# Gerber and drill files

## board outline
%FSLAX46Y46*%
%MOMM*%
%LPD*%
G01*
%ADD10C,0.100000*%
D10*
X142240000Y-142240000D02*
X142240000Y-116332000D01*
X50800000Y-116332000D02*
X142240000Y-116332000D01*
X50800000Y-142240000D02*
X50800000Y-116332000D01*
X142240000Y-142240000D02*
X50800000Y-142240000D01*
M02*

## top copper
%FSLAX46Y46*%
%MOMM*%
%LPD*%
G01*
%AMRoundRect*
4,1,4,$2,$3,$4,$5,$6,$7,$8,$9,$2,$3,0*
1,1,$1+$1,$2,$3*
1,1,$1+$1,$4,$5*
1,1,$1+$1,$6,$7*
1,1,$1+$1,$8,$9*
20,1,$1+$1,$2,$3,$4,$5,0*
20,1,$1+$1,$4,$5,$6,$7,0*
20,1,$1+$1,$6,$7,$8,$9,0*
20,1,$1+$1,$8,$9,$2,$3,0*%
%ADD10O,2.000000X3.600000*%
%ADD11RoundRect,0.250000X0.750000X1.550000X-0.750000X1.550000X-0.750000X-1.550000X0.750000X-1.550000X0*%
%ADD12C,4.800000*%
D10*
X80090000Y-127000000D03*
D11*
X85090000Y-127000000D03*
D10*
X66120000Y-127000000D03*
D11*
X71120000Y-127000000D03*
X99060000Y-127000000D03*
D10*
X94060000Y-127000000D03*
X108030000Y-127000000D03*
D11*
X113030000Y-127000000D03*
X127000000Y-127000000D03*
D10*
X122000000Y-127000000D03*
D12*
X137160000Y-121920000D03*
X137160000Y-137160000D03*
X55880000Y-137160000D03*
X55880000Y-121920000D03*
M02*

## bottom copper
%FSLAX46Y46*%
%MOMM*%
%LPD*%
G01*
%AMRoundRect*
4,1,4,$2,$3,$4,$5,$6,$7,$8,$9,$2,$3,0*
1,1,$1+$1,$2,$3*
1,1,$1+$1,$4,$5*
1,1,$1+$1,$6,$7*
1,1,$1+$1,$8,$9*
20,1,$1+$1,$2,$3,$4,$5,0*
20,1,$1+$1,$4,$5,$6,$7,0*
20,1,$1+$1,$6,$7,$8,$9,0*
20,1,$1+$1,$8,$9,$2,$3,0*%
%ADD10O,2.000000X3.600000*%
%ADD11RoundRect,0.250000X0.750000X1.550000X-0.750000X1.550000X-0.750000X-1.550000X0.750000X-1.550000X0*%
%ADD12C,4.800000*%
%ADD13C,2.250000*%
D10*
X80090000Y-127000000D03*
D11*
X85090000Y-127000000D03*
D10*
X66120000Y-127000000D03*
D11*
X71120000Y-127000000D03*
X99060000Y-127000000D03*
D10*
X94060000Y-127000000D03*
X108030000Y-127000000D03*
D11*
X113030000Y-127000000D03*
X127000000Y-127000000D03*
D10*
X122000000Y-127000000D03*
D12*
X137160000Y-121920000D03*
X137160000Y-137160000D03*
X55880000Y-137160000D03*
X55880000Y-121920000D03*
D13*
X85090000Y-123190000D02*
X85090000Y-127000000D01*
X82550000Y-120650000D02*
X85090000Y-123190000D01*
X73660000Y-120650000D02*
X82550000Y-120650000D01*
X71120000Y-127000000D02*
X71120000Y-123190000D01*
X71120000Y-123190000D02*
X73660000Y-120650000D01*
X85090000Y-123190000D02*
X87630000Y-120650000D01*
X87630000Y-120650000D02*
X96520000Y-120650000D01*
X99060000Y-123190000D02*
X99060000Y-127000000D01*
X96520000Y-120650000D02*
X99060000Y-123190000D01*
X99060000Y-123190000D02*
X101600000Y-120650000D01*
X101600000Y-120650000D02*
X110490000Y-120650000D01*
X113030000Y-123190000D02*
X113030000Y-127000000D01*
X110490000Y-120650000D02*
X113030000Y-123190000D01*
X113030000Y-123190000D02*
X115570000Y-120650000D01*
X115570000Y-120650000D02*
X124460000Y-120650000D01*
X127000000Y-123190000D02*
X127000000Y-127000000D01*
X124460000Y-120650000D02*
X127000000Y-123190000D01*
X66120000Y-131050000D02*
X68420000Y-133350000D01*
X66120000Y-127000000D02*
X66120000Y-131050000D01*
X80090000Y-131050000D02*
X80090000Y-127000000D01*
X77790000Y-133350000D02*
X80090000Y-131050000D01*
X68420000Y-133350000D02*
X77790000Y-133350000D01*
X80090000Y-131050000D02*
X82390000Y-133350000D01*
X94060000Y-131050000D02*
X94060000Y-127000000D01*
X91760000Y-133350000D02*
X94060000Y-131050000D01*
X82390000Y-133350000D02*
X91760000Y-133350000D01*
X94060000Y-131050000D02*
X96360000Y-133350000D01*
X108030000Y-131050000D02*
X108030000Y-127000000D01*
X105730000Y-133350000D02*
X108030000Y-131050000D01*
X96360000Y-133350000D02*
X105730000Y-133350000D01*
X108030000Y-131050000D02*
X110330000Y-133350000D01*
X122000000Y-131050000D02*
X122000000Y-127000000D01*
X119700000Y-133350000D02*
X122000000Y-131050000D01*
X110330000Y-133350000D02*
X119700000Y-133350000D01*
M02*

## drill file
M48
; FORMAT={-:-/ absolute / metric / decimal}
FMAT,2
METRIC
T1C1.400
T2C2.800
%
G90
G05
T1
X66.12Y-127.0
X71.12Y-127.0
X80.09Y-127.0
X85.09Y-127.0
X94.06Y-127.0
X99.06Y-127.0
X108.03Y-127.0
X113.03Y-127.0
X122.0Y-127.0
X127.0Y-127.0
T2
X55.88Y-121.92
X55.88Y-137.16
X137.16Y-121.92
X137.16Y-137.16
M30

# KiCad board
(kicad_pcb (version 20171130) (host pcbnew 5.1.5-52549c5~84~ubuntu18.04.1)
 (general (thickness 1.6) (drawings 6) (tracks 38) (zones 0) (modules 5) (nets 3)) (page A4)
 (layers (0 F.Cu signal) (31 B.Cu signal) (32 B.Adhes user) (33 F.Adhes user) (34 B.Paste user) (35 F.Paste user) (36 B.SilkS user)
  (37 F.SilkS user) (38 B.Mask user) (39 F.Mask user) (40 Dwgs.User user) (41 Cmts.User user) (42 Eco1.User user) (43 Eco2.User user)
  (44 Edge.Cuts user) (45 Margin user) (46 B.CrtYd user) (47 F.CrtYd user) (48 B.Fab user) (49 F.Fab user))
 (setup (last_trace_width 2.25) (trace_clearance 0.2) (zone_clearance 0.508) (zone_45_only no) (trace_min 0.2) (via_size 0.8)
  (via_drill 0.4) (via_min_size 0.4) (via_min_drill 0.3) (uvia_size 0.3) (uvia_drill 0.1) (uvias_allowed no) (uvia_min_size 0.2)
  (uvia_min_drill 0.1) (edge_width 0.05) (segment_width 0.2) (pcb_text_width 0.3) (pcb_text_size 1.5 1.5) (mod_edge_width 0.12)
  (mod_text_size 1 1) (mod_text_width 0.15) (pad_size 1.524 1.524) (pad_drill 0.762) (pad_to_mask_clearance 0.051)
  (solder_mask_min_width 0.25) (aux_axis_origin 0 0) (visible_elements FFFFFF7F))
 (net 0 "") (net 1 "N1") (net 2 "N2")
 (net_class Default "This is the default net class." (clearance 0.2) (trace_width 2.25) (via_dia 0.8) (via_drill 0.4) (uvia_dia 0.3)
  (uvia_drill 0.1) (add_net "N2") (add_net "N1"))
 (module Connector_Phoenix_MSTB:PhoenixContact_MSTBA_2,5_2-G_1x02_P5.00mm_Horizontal (layer F.Cu) (at 85.09 127 180)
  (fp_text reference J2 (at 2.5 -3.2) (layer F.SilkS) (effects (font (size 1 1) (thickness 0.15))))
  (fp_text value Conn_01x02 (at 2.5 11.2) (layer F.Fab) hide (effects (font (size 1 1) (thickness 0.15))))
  (pad 2 thru_hole oval (at 5 0 180) (size 2 3.6) (drill 1.4) (layers *.Cu *.Mask) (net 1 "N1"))
  (pad 1 thru_hole roundrect (at 0 0 180) (size 2 3.6) (drill 1.4) (layers *.Cu *.Mask) (roundrect_rratio 0.125) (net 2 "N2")))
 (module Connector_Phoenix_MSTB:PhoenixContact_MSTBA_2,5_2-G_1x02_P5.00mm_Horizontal (layer F.Cu) (at 71.12 127 180)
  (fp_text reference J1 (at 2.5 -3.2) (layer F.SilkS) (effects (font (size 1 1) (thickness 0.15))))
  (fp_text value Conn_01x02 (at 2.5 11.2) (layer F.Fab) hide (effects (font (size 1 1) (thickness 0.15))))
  (pad 2 thru_hole oval (at 5 0 180) (size 2 3.6) (drill 1.4) (layers *.Cu *.Mask) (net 1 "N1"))
  (pad 1 thru_hole roundrect (at 0 0 180) (size 2 3.6) (drill 1.4) (layers *.Cu *.Mask) (roundrect_rratio 0.125) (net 2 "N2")))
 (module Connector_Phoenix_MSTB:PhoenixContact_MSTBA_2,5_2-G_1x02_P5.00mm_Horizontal (layer F.Cu) (at 99.06 127 180)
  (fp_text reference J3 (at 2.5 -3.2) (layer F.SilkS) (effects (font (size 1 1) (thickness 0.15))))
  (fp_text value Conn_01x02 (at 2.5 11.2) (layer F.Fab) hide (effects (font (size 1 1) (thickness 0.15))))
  (pad 1 thru_hole roundrect (at 0 0 180) (size 2 3.6) (drill 1.4) (layers *.Cu *.Mask) (roundrect_rratio 0.125) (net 2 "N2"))
  (pad 2 thru_hole oval (at 5 0 180) (size 2 3.6) (drill 1.4) (layers *.Cu *.Mask) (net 1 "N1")))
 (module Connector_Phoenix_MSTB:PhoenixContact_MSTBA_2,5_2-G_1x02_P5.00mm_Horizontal (layer F.Cu) (at 113.03 127 180)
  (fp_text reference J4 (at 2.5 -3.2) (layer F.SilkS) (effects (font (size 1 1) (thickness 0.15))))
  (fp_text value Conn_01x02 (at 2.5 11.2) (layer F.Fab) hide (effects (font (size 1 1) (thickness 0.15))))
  (pad 2 thru_hole oval (at 5 0 180) (size 2 3.6) (drill 1.4) (layers *.Cu *.Mask) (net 1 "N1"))
  (pad 1 thru_hole roundrect (at 0 0 180) (size 2 3.6) (drill 1.4) (layers *.Cu *.Mask) (roundrect_rratio 0.125) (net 2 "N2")))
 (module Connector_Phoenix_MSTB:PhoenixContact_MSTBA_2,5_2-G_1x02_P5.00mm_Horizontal (layer F.Cu) (at 127 127 180)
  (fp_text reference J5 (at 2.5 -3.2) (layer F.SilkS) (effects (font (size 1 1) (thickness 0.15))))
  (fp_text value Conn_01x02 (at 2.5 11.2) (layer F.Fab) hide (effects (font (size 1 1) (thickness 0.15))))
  (pad 1 thru_hole roundrect (at 0 0 180) (size 2 3.6) (drill 1.4) (layers *.Cu *.Mask) (roundrect_rratio 0.125) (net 2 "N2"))
  (pad 2 thru_hole oval (at 5 0 180) (size 2 3.6) (drill 1.4) (layers *.Cu *.Mask) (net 1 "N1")))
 (gr_line (start 142.24 142.24) (end 142.24 116.332) (layer Edge.Cuts) (width 0.1))
 (gr_line (start 50.8 116.332) (end 142.24 116.332) (layer Edge.Cuts) (width 0.1))
 (gr_line (start 50.8 142.24) (end 50.8 116.332) (layer Edge.Cuts) (width 0.1))
 (gr_line (start 142.24 142.24) (end 50.8 142.24) (layer Edge.Cuts) (width 0.1))
 (via (at 137.16 121.92) (size 4.8) (drill 2.8) (layers F.Cu B.Cu) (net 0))
 (via (at 137.16 137.16) (size 4.8) (drill 2.8) (layers F.Cu B.Cu) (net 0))
 (via (at 55.88 137.16) (size 4.8) (drill 2.8) (layers F.Cu B.Cu) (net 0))
 (via (at 55.88 121.92) (size 4.8) (drill 2.8) (layers F.Cu B.Cu) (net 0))
 (segment (start 85.09 123.19) (end 85.09 127) (width 2.25) (layer B.Cu) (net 2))
 (segment (start 82.55 120.65) (end 85.09 123.19) (width 2.25) (layer B.Cu) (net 2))
 (segment (start 73.66 120.65) (end 82.55 120.65) (width 2.25) (layer B.Cu) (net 2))
 (segment (start 71.12 127) (end 71.12 123.19) (width 2.25) (layer B.Cu) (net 2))
 (segment (start 71.12 123.19) (end 73.66 120.65) (width 2.25) (layer B.Cu) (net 2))
 (segment (start 85.09 123.19) (end 87.63 120.65) (width 2.25) (layer B.Cu) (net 2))
 (segment (start 87.63 120.65) (end 96.52 120.65) (width 2.25) (layer B.Cu) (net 2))
 (segment (start 99.06 123.19) (end 99.06 127) (width 2.25) (layer B.Cu) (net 2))
 (segment (start 96.52 120.65) (end 99.06 123.19) (width 2.25) (layer B.Cu) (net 2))
 (segment (start 99.06 123.19) (end 101.6 120.65) (width 2.25) (layer B.Cu) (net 2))
 (segment (start 101.6 120.65) (end 110.49 120.65) (width 2.25) (layer B.Cu) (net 2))
 (segment (start 113.03 123.19) (end 113.03 127) (width 2.25) (layer B.Cu) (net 2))
 (segment (start 110.49 120.65) (end 113.03 123.19) (width 2.25) (layer B.Cu) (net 2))
 (segment (start 113.03 123.19) (end 115.57 120.65) (width 2.25) (layer B.Cu) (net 2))
 (segment (start 115.57 120.65) (end 124.46 120.65) (width 2.25) (layer B.Cu) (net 2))
 (segment (start 127 123.19) (end 127 127) (width 2.25) (layer B.Cu) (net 2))
 (segment (start 124.46 120.65) (end 127 123.19) (width 2.25) (layer B.Cu) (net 2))
 (segment (start 66.12 131.05) (end 68.42 133.35) (width 2.25) (layer B.Cu) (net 1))
 (segment (start 66.12 127) (end 66.12 131.05) (width 2.25) (layer B.Cu) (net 1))
 (segment (start 80.09 131.05) (end 80.09 127) (width 2.25) (layer B.Cu) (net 1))
 (segment (start 77.79 133.35) (end 80.09 131.05) (width 2.25) (layer B.Cu) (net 1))
 (segment (start 68.42 133.35) (end 77.79 133.35) (width 2.25) (layer B.Cu) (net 1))
 (segment (start 80.09 131.05) (end 82.39 133.35) (width 2.25) (layer B.Cu) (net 1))
 (segment (start 94.06 131.05) (end 94.06 127) (width 2.25) (layer B.Cu) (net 1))
 (segment (start 91.76 133.35) (end 94.06 131.05) (width 2.25) (layer B.Cu) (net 1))
 (segment (start 82.39 133.35) (end 91.76 133.35) (width 2.25) (layer B.Cu) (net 1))
 (segment (start 94.06 131.05) (end 96.36 133.35) (width 2.25) (layer B.Cu) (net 1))
 (segment (start 108.03 131.05) (end 108.03 127) (width 2.25) (layer B.Cu) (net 1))
 (segment (start 105.73 133.35) (end 108.03 131.05) (width 2.25) (layer B.Cu) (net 1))
 (segment (start 96.36 133.35) (end 105.73 133.35) (width 2.25) (layer B.Cu) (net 1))
 (segment (start 108.03 131.05) (end 110.33 133.35) (width 2.25) (layer B.Cu) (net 1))
 (segment (start 122 131.05) (end 122 127) (width 2.25) (layer B.Cu) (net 1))
 (segment (start 119.7 133.35) (end 122 131.05) (width 2.25) (layer B.Cu) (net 1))
 (segment (start 110.33 133.35) (end 119.7 133.35) (width 2.25) (layer B.Cu) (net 1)))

